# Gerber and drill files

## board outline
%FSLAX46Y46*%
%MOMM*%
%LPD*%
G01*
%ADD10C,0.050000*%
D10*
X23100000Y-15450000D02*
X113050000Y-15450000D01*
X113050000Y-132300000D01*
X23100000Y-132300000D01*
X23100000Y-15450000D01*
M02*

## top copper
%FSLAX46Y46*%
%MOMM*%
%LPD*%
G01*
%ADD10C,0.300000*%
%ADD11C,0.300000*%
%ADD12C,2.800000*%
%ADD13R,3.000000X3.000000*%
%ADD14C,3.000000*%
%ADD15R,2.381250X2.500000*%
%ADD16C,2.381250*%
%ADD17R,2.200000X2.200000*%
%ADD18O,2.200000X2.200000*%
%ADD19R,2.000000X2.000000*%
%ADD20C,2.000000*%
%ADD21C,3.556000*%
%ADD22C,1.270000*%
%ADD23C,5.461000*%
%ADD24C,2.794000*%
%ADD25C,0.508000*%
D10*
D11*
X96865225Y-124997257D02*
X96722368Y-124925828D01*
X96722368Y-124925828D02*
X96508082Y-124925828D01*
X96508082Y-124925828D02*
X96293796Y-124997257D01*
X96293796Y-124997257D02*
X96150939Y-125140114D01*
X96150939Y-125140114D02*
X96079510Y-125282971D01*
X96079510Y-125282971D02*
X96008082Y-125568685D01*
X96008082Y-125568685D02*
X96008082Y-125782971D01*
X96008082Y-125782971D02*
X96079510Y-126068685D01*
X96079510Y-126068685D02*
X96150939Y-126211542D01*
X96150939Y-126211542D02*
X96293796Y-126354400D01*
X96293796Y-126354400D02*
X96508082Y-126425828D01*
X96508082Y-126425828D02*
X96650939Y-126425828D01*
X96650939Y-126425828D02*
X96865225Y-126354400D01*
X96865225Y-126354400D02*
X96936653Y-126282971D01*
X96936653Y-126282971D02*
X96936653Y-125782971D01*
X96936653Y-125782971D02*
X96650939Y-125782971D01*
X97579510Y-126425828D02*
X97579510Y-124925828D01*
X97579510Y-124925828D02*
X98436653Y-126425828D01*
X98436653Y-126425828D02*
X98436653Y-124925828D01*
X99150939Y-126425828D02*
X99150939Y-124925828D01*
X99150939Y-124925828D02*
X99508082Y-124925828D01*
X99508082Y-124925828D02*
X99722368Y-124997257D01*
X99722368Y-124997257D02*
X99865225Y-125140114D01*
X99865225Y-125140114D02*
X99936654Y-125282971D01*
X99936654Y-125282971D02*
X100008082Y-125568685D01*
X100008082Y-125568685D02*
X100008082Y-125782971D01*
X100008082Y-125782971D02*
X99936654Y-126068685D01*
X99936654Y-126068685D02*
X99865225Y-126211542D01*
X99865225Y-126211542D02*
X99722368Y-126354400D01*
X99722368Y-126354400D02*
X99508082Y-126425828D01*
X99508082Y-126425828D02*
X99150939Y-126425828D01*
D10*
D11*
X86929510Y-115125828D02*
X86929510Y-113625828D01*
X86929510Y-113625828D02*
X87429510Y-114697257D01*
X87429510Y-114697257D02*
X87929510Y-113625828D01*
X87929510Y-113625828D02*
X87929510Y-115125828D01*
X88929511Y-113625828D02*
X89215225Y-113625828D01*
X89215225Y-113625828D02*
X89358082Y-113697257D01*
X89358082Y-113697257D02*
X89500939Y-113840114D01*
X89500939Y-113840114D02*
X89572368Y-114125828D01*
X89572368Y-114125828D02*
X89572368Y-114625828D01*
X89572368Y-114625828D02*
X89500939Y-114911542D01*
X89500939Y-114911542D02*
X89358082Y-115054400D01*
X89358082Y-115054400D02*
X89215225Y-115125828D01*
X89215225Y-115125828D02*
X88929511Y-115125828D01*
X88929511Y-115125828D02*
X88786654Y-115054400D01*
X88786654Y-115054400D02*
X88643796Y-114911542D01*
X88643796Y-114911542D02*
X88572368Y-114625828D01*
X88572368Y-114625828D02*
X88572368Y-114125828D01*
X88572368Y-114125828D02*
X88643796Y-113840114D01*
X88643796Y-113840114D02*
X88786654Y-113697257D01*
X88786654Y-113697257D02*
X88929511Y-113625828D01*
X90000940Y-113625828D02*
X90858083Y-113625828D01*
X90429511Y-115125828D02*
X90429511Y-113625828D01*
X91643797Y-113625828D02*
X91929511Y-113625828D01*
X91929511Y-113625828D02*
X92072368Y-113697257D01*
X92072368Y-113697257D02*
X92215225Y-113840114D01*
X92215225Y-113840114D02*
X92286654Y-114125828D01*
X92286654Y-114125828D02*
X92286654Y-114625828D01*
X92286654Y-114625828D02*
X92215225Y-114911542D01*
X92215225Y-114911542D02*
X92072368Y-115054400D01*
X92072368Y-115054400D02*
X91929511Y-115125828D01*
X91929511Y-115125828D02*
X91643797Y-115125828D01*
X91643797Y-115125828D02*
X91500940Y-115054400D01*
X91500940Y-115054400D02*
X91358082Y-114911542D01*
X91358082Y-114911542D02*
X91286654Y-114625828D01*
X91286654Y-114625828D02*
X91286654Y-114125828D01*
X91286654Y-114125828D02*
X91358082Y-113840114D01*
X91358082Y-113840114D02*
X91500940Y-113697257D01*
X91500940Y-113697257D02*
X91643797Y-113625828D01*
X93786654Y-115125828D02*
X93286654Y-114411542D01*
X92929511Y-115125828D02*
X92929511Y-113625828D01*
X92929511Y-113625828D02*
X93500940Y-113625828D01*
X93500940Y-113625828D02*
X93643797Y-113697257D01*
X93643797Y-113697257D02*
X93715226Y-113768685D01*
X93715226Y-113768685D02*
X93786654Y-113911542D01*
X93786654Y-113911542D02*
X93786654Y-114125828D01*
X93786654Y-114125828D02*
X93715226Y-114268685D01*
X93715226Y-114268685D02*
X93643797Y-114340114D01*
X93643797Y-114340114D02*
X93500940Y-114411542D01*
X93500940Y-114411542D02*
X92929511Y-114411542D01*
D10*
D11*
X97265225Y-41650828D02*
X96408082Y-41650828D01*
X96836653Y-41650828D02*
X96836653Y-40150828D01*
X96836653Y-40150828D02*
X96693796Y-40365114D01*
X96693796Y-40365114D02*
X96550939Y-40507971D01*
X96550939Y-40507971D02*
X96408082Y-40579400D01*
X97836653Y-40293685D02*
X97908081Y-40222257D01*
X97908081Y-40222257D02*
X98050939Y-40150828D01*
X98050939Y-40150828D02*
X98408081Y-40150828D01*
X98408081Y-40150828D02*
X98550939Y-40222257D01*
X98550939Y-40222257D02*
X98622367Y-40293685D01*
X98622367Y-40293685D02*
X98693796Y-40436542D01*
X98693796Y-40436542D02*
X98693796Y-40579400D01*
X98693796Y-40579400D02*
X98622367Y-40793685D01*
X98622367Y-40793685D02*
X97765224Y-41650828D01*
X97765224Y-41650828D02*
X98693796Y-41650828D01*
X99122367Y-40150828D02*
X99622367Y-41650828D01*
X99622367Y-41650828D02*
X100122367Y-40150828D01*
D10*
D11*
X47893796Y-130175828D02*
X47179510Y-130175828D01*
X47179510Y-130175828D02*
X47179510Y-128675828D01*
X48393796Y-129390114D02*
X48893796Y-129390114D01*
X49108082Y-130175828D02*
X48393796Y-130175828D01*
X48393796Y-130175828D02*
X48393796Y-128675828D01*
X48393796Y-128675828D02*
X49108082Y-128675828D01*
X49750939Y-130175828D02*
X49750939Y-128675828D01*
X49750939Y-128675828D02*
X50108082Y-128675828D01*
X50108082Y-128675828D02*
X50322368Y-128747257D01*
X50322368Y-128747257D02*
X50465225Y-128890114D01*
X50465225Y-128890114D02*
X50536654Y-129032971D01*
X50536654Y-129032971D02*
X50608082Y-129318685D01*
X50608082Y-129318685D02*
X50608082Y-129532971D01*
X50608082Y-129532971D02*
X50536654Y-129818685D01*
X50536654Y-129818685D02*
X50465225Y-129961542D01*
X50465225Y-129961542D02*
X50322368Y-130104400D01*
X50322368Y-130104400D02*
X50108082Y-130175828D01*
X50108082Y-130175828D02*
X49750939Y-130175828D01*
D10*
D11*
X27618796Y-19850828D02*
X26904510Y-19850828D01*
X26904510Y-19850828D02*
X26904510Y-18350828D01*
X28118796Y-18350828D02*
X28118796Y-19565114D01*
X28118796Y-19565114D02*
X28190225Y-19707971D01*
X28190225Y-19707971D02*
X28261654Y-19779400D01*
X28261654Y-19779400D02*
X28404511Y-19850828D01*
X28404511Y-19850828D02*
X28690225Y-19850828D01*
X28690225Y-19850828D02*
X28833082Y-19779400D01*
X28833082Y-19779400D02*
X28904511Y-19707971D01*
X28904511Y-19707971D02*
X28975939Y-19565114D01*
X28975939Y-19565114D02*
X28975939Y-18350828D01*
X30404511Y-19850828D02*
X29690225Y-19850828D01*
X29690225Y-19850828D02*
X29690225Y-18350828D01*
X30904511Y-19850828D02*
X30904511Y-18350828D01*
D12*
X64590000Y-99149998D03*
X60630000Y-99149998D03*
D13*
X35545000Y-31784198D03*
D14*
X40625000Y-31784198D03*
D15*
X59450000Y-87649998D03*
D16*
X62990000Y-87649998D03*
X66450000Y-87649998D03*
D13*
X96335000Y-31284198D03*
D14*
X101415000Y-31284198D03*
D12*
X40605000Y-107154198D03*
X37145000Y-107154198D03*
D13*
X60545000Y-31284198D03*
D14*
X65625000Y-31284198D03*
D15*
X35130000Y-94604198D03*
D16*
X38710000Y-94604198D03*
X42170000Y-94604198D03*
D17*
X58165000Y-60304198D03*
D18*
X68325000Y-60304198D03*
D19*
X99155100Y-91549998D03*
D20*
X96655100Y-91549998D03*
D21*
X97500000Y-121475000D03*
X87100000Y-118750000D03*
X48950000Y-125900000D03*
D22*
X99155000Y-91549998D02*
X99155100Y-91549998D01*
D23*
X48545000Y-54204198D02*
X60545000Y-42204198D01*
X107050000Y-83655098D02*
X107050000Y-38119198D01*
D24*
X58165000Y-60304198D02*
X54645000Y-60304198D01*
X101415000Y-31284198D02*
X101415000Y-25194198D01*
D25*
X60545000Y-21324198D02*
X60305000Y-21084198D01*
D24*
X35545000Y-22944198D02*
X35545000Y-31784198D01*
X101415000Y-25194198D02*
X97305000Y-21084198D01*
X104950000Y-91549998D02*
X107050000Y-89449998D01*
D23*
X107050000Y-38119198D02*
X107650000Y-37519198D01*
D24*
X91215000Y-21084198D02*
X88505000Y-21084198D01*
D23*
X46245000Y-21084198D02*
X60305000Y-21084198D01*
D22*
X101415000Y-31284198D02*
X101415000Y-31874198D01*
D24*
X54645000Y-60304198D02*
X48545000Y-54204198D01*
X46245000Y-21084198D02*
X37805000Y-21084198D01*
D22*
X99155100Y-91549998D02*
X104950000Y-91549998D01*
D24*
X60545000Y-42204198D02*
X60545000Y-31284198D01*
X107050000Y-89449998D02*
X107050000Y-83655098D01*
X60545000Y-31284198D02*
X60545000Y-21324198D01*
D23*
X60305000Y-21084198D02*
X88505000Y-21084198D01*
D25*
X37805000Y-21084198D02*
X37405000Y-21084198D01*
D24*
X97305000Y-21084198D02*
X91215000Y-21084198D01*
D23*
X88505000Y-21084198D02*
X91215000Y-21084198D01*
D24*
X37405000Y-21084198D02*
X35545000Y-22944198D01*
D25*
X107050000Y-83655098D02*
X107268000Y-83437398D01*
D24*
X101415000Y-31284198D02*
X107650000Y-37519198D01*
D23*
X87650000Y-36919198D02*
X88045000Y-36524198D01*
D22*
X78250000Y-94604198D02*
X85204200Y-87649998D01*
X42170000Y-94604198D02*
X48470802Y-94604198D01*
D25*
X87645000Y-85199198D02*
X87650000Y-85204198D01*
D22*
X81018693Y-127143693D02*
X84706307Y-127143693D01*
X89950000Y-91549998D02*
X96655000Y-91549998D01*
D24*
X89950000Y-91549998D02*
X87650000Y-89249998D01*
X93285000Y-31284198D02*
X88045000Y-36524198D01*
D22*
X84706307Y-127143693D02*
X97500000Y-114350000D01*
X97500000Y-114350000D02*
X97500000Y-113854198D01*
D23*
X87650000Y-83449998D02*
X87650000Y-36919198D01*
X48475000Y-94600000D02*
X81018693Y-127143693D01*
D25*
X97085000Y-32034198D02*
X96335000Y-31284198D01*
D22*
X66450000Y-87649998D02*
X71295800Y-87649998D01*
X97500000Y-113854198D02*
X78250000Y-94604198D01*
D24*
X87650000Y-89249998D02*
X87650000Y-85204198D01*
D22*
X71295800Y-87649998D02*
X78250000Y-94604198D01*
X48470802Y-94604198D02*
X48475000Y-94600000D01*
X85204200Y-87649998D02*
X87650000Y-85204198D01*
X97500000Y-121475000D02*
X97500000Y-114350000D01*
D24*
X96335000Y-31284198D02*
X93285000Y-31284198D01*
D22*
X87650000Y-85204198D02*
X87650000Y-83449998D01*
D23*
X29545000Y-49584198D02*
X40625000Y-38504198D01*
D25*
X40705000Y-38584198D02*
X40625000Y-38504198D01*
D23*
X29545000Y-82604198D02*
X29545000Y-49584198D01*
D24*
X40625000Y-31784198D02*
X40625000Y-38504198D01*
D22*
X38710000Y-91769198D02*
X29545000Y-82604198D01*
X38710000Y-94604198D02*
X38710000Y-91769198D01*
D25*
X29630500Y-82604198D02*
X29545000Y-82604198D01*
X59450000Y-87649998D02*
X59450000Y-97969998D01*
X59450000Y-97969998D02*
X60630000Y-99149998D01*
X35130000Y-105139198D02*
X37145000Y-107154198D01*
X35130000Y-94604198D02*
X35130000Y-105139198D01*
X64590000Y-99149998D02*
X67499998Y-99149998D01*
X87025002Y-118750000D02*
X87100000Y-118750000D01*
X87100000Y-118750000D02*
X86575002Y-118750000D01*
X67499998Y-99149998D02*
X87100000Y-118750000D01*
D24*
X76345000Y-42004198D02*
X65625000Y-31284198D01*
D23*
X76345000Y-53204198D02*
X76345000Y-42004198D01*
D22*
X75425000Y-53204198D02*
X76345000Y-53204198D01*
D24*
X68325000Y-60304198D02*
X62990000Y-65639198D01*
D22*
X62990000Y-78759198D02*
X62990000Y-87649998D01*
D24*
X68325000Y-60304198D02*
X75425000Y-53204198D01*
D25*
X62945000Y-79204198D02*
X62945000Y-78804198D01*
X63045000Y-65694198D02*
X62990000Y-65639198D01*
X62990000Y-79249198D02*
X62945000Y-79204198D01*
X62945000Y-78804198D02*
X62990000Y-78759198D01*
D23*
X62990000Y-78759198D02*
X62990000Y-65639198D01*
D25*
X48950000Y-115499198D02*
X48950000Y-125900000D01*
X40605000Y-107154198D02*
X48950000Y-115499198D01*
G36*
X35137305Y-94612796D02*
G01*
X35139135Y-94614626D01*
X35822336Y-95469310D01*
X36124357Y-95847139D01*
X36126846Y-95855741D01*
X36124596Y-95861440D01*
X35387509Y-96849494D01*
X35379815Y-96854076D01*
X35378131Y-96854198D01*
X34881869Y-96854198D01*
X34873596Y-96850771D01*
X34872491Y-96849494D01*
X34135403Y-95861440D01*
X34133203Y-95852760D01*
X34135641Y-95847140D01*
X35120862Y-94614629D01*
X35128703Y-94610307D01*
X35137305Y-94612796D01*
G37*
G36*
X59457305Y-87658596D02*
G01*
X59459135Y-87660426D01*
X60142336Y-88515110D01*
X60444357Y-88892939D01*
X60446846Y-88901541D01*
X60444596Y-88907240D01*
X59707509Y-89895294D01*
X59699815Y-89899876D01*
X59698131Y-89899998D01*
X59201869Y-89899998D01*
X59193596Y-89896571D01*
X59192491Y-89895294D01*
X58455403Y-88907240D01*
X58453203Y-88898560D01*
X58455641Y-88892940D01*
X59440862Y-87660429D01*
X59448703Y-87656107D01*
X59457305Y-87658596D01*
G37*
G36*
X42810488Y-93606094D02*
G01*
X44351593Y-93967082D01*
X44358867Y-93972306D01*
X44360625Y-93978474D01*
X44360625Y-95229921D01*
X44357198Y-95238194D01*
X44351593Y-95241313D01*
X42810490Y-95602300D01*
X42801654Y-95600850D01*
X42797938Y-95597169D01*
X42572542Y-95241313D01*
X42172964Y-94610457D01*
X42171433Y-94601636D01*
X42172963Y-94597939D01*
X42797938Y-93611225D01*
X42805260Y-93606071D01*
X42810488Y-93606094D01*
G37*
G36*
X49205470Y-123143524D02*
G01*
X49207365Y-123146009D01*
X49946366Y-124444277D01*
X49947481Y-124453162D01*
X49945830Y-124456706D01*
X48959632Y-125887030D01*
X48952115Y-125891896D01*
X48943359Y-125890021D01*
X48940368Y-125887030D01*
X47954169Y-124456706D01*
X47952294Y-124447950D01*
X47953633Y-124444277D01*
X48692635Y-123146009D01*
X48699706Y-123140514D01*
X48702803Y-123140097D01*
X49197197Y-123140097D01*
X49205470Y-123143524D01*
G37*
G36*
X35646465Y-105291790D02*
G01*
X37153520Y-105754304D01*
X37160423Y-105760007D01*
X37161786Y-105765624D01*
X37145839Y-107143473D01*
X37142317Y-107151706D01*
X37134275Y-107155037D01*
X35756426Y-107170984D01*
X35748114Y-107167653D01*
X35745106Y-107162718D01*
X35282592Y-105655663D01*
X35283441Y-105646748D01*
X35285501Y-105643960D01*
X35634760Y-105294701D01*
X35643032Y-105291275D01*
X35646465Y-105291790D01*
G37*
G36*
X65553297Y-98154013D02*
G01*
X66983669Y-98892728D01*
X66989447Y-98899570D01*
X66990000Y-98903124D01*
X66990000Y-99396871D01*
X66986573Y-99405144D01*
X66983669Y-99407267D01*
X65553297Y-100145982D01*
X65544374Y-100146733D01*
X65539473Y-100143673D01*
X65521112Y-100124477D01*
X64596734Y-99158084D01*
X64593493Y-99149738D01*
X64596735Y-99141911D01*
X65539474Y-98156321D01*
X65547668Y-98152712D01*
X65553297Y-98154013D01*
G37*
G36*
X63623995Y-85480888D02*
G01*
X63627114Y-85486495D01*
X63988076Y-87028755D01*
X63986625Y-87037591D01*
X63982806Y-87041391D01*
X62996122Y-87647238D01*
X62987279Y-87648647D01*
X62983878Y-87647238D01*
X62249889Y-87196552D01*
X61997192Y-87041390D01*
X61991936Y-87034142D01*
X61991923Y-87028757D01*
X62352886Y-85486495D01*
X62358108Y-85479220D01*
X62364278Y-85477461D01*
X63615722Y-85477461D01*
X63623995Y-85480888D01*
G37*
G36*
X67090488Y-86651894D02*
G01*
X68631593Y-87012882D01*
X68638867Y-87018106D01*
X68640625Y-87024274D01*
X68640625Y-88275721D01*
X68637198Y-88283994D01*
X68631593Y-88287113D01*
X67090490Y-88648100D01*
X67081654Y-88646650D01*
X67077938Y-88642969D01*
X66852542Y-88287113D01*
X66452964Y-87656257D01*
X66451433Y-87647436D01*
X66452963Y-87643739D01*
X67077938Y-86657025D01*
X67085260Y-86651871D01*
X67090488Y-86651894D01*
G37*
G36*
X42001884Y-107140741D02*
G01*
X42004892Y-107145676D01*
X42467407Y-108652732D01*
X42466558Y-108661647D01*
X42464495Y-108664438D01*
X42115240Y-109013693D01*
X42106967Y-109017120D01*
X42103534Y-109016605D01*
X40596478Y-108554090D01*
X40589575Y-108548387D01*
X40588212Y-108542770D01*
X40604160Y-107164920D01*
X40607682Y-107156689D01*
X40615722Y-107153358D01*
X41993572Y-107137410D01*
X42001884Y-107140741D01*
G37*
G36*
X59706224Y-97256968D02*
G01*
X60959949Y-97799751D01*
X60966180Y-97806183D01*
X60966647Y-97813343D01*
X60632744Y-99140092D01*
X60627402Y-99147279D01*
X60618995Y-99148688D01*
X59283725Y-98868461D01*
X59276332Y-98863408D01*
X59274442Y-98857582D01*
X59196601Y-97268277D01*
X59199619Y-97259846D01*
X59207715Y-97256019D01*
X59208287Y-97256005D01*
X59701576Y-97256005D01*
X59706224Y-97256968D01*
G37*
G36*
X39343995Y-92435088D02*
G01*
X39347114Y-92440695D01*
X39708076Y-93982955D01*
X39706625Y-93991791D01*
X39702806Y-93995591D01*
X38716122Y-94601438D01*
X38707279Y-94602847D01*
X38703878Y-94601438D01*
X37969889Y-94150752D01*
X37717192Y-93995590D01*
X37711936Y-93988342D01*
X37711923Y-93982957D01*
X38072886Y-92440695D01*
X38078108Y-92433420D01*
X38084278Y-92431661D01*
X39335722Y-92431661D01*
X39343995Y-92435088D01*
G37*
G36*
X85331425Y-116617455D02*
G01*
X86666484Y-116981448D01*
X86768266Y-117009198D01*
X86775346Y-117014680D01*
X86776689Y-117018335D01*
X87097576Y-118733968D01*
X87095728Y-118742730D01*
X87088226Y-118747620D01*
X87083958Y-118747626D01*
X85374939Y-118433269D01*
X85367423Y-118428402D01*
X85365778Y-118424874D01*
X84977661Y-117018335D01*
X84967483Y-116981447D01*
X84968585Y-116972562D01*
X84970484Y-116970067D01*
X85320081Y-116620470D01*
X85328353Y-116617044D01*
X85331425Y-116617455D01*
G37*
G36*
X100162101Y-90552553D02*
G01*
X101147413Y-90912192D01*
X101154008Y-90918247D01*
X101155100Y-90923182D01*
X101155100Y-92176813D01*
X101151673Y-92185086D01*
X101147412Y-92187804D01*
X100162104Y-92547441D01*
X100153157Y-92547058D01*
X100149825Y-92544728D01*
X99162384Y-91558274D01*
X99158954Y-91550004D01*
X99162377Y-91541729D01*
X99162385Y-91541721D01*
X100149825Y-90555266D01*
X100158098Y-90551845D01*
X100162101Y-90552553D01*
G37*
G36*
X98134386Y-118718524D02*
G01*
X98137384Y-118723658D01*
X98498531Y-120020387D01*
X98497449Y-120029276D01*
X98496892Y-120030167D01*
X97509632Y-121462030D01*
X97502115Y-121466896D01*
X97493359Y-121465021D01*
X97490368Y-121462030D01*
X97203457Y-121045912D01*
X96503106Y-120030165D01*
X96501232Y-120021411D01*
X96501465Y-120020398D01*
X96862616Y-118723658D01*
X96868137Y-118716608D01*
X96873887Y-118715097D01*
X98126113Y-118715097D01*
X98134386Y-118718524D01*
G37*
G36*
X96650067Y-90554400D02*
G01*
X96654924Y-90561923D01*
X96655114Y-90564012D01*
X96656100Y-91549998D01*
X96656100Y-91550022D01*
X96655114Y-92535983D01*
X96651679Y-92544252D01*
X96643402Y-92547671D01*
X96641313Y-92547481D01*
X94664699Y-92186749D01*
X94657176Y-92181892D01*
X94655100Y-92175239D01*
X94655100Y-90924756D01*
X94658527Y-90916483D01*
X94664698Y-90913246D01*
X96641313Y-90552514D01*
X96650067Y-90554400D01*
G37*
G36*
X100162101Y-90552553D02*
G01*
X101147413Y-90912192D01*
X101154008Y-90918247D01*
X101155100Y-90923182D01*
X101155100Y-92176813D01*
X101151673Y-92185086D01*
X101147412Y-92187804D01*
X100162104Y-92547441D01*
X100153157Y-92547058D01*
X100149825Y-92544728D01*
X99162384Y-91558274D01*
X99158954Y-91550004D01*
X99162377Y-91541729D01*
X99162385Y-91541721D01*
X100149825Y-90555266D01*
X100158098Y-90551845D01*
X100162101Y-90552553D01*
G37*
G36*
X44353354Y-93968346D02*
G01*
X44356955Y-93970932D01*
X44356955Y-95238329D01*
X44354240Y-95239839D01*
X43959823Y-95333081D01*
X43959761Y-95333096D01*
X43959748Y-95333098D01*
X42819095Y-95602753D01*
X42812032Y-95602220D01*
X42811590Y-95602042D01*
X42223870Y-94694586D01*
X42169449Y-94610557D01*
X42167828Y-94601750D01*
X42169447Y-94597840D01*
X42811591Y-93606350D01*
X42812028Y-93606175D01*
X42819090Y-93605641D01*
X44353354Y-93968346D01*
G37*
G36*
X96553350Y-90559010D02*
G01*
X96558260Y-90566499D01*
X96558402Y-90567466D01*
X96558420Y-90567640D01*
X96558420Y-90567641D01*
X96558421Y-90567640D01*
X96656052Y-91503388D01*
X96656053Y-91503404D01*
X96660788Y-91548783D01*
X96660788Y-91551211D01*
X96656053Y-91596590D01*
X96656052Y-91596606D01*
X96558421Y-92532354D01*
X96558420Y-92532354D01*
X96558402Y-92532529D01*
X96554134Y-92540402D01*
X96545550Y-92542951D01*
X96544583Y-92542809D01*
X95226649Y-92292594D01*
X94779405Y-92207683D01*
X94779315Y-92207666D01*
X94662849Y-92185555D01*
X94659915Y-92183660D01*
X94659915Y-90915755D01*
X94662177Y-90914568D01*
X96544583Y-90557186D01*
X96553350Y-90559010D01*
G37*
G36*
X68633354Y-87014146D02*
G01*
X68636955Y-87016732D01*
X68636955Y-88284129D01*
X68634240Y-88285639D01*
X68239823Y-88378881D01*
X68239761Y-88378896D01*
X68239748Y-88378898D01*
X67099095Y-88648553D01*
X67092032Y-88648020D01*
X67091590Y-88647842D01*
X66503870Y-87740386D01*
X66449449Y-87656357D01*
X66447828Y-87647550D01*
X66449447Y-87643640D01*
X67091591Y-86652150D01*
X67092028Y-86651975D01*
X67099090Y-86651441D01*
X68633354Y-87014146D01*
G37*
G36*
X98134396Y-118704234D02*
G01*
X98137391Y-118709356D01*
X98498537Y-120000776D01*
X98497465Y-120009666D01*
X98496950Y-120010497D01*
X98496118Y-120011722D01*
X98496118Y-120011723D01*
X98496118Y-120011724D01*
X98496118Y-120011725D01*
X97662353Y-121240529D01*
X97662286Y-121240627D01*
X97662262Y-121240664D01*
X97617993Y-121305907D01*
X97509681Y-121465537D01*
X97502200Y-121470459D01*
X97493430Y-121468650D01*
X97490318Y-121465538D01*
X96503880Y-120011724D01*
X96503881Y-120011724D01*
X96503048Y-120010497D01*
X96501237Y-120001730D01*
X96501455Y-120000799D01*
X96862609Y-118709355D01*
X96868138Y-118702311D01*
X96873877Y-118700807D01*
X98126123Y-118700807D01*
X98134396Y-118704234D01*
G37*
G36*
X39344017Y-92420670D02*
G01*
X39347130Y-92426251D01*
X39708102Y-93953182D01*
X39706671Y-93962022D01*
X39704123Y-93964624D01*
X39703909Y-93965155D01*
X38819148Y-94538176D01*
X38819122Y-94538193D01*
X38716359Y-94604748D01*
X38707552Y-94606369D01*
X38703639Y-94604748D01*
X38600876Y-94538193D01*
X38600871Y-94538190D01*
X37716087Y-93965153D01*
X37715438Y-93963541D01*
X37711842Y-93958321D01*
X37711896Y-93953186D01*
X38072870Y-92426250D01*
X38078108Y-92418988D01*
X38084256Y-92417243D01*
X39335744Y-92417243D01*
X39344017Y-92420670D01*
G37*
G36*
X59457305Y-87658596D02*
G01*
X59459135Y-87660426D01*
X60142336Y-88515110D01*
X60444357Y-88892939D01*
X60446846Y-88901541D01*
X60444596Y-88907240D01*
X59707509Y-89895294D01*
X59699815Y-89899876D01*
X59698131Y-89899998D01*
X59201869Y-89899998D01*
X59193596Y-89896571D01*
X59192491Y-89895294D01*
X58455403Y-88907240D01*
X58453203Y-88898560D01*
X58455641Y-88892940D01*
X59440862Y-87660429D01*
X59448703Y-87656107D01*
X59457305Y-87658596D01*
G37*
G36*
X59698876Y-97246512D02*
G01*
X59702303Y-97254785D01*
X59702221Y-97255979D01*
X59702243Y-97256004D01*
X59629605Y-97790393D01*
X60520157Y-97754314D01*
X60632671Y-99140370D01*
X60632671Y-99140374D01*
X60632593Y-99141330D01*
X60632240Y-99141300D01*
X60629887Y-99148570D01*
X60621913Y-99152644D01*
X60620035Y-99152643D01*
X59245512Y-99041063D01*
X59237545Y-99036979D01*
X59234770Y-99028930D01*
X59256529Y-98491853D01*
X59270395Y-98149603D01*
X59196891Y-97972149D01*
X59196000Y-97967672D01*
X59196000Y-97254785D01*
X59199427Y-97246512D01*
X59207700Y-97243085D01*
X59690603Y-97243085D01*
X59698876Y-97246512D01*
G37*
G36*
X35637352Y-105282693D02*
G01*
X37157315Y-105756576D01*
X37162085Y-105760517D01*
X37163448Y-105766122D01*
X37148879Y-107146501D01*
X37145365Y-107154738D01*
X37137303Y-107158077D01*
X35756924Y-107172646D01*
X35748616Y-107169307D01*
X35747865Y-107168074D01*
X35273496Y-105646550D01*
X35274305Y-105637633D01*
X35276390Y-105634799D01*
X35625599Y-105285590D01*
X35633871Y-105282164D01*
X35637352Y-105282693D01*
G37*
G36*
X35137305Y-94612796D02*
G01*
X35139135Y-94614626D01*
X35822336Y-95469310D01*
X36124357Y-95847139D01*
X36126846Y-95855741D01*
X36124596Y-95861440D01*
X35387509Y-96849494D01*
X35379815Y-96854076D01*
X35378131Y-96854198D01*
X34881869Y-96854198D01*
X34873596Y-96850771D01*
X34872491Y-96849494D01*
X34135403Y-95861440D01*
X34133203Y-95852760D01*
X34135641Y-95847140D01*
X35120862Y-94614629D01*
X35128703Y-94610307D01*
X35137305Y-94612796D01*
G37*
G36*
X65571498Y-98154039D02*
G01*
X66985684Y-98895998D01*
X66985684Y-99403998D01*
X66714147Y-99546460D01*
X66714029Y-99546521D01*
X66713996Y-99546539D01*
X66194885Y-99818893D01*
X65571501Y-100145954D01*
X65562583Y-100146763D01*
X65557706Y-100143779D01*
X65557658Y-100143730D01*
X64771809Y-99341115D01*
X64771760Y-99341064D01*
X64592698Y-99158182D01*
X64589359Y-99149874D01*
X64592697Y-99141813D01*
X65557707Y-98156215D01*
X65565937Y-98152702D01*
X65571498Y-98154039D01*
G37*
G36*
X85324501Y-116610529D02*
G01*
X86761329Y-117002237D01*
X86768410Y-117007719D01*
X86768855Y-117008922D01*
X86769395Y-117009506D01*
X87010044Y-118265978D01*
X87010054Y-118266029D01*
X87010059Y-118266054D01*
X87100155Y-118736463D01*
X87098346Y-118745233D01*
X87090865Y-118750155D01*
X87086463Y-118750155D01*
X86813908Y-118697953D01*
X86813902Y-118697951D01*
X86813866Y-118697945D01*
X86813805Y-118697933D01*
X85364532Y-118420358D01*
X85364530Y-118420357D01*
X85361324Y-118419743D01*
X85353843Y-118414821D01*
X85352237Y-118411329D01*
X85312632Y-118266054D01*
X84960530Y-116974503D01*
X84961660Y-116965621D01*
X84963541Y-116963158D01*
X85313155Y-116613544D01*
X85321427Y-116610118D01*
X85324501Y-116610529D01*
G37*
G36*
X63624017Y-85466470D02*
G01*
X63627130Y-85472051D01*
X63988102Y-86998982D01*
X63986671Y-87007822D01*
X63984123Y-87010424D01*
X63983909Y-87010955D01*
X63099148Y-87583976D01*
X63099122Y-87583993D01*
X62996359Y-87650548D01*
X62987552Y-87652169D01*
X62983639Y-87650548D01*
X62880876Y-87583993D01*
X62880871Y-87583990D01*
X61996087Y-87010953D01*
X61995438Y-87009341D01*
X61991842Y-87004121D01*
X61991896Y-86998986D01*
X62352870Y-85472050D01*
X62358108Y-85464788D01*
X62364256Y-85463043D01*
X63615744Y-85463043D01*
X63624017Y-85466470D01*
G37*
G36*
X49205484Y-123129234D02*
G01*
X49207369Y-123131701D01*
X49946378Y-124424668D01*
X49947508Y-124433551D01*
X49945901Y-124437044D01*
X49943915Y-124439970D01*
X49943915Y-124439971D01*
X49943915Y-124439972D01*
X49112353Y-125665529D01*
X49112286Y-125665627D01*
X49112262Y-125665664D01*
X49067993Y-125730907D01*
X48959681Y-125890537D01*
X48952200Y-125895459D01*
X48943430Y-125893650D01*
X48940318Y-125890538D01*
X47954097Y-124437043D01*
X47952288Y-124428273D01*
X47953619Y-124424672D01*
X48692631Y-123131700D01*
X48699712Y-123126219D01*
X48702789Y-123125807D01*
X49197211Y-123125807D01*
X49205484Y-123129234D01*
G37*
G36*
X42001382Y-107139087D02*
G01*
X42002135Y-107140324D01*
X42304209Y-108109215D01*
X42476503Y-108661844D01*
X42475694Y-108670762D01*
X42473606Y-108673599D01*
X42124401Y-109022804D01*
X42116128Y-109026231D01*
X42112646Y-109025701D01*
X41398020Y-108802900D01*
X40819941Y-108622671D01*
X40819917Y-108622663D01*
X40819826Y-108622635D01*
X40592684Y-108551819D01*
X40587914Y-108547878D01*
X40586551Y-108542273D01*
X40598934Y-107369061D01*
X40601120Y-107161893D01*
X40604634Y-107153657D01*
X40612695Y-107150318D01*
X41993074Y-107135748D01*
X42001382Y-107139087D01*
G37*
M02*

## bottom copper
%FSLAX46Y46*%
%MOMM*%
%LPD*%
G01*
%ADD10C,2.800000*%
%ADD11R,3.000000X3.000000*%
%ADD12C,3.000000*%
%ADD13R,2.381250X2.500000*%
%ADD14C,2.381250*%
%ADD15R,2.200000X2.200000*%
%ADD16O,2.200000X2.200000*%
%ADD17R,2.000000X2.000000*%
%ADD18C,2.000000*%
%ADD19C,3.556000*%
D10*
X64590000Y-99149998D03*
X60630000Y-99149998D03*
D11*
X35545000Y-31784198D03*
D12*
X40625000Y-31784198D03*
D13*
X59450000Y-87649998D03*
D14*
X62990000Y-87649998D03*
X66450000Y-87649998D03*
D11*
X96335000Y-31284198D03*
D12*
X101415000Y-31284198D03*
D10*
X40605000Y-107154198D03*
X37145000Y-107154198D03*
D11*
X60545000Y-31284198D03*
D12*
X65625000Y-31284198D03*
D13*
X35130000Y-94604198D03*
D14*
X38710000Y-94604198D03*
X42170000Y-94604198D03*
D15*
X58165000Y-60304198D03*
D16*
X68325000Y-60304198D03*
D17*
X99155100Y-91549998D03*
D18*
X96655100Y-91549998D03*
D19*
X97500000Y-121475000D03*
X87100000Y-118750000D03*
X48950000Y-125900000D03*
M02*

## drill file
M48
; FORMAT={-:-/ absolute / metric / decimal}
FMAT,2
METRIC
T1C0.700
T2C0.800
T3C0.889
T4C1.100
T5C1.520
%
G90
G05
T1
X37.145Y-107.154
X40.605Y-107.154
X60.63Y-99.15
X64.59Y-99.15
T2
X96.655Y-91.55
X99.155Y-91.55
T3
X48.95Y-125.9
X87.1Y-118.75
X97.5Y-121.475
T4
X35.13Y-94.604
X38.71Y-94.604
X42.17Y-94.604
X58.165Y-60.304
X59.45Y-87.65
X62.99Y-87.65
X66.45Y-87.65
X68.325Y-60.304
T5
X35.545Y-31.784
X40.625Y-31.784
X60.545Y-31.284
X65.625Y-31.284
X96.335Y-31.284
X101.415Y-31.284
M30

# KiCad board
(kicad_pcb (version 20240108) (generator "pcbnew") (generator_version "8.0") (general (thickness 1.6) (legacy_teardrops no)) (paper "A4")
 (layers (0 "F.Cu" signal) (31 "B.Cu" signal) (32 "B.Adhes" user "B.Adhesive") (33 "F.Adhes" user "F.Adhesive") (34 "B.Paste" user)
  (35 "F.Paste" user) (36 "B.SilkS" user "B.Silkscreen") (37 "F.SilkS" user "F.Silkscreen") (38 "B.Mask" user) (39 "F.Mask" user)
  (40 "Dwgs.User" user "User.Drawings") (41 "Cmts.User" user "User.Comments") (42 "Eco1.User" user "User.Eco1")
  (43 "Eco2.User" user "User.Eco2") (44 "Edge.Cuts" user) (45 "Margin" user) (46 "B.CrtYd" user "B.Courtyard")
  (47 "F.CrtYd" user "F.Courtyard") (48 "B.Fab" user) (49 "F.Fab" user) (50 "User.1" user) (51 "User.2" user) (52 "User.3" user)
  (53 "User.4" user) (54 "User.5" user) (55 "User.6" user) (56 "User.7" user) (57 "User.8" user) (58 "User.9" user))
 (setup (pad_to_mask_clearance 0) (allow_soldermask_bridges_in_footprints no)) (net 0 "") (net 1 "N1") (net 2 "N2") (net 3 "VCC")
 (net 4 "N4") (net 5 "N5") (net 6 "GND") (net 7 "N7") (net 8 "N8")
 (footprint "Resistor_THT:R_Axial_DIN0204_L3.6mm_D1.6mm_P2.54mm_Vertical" (layer "F.Cu") (at 63.17 99.149998 180)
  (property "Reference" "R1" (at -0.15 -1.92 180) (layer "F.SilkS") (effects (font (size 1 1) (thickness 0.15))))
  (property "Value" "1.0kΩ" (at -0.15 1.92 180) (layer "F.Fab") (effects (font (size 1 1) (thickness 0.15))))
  (pad "1" thru_hole circle (at -1.42 0 180) (size 2.8 2.8) (drill 0.7) (layers "*.Cu" "*.Mask") (remove_unused_layers no) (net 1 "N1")
   (teardrops (best_length_ratio 0.5) (max_length 1) (best_width_ratio 1) (max_width 2) (curve_points 0) (filter_ratio 0.9) (enabled yes)
    (allow_two_segments yes) (prefer_zone_connections yes)))
  (pad "2" thru_hole circle (at 2.54 0 180) (size 2.8 2.8) (drill 0.7) (layers "*.Cu" "*.Mask") (remove_unused_layers no) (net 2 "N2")
   (teardrops (best_length_ratio 0.5) (max_length 1) (best_width_ratio 1) (max_width 2) (curve_points 0) (filter_ratio 0.9) (enabled yes)
    (allow_two_segments yes) (prefer_zone_connections yes))))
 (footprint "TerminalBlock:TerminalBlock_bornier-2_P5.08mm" (layer "F.Cu") (at 35.545 31.784198)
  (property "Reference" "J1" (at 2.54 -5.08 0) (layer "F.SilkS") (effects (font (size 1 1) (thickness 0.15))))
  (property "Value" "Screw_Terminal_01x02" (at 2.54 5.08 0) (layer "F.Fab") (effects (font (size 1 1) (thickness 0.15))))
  (pad "1" thru_hole rect (at 0 0) (size 3 3) (drill 1.52) (layers "*.Cu" "*.Mask") (remove_unused_layers no) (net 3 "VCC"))
  (pad "2" thru_hole circle (at 5.08 0) (size 3 3) (drill 1.52) (layers "*.Cu" "*.Mask") (remove_unused_layers no) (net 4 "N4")))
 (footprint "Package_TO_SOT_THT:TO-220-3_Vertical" (layer "F.Cu") (at 60.45 87.649998)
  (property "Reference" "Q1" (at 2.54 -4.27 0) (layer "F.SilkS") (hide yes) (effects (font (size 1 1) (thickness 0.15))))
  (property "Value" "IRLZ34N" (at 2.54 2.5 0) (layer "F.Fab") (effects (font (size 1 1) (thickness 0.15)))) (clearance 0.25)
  (pad "1" thru_hole rect (at -1 0) (size 2.38125 2.5) (drill 1.1) (layers "*.Cu" "*.Mask") (remove_unused_layers no) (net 2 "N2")
   (teardrops (best_length_ratio 0.5) (max_length 1) (best_width_ratio 1) (max_width 2) (curve_points 0) (filter_ratio 0.9) (enabled yes)
    (allow_two_segments yes) (prefer_zone_connections yes)))
  (pad "2" thru_hole circle (at 2.54 0) (size 2.38125 2.38125) (drill 1.1) (layers "*.Cu" "*.Mask") (remove_unused_layers no) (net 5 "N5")
   (clearance 0.2)
   (teardrops (best_length_ratio 0.5) (max_length 1) (best_width_ratio 1) (max_width 2) (curve_points 0) (filter_ratio 0.9) (enabled yes)
    (allow_two_segments yes) (prefer_zone_connections yes)))
  (pad "3" thru_hole circle (at 6 0) (size 2.38125 2.38125) (drill 1.1) (layers "*.Cu" "*.Mask") (remove_unused_layers no) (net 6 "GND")
   (teardrops (best_length_ratio 0.5) (max_length 1) (best_width_ratio 1) (max_width 2) (curve_points 0) (filter_ratio 0.9) (enabled yes)
    (allow_two_segments yes) (prefer_zone_connections yes))))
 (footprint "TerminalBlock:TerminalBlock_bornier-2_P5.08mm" (layer "F.Cu") (at 96.335 31.284198)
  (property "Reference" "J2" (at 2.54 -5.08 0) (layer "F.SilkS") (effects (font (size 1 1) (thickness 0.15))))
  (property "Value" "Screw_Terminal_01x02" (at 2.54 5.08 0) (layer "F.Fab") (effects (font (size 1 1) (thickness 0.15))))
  (pad "1" thru_hole rect (at 0 0) (size 3 3) (drill 1.52) (layers "*.Cu" "*.Mask") (remove_unused_layers no) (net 6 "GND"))
  (pad "2" thru_hole circle (at 5.08 0) (size 3 3) (drill 1.52) (layers "*.Cu" "*.Mask") (remove_unused_layers no) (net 3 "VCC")))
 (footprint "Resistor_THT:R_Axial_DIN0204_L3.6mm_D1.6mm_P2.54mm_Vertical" (layer "F.Cu") (at 39.685 107.154198 180)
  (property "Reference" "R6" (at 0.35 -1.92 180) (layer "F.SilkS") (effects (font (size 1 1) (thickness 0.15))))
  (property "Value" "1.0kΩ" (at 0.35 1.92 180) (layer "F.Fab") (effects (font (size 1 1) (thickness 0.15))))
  (pad "1" thru_hole circle (at -0.92 0 180) (size 2.8 2.8) (drill 0.7) (layers "*.Cu" "*.Mask") (remove_unused_layers no) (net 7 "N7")
   (teardrops (best_length_ratio 0.5) (max_length 1) (best_width_ratio 1) (max_width 2) (curve_points 0) (filter_ratio 0.9) (enabled yes)
    (allow_two_segments yes) (prefer_zone_connections yes)))
  (pad "2" thru_hole circle (at 2.54 0 180) (size 2.8 2.8) (drill 0.7) (layers "*.Cu" "*.Mask") (remove_unused_layers no) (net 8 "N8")
   (teardrops (best_length_ratio 0.5) (max_length 1) (best_width_ratio 1) (max_width 2) (curve_points 0) (filter_ratio 0.9) (enabled yes)
    (allow_two_segments yes) (prefer_zone_connections yes))))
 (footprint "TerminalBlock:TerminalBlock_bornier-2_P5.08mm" (layer "F.Cu") (at 60.545 31.284198)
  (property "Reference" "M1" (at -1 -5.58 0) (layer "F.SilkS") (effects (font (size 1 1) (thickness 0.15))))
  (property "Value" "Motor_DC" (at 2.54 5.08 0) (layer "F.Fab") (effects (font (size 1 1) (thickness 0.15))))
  (pad "1" thru_hole rect (at 0 0) (size 3 3) (drill 1.52) (layers "*.Cu" "*.Mask") (remove_unused_layers no) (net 3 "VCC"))
  (pad "2" thru_hole circle (at 5.08 0) (size 3 3) (drill 1.52) (layers "*.Cu" "*.Mask") (remove_unused_layers no) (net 5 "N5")))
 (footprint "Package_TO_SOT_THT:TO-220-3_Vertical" (layer "F.Cu") (at 37.17 94.604198)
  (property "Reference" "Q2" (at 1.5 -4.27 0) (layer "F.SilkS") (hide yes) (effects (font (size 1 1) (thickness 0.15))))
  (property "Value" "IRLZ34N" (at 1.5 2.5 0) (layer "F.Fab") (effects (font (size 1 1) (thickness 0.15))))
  (pad "1" thru_hole rect (at -2.04 0) (size 2.38125 2.5) (drill 1.1) (layers "*.Cu" "*.Mask") (remove_unused_layers no) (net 8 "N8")
   (teardrops (best_length_ratio 0.5) (max_length 1) (best_width_ratio 1) (max_width 2) (curve_points 0) (filter_ratio 0.9) (enabled yes)
    (allow_two_segments yes) (prefer_zone_connections yes)))
  (pad "2" thru_hole circle (at 1.54 0) (size 2.38125 2.38125) (drill 1.1) (layers "*.Cu" "*.Mask") (remove_unused_layers no) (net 4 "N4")
   (teardrops (best_length_ratio 0.5) (max_length 1) (best_width_ratio 1) (max_width 2) (curve_points 0) (filter_ratio 0.9) (enabled yes)
    (allow_two_segments yes) (prefer_zone_connections yes)))
  (pad "3" thru_hole circle (at 5 0) (size 2.38125 2.38125) (drill 1.1) (layers "*.Cu" "*.Mask") (remove_unused_layers no) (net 6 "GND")
   (teardrops (best_length_ratio 0.5) (max_length 1) (best_width_ratio 1) (max_width 2) (curve_points 0) (filter_ratio 0.9) (enabled yes)
    (allow_two_segments yes) (prefer_zone_connections yes))))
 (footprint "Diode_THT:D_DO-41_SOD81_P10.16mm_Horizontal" (layer "F.Cu") (at 58.165 60.304198)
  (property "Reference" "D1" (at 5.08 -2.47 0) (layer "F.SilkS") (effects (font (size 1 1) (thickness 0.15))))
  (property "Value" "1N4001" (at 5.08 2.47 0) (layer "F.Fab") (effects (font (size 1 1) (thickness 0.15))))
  (pad "1" thru_hole rect (at 0 0) (size 2.2 2.2) (drill 1.1) (layers "*.Cu" "*.Mask") (remove_unused_layers no) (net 3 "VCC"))
  (pad "2" thru_hole oval (at 10.16 0) (size 2.2 2.2) (drill 1.1) (layers "*.Cu" "*.Mask") (remove_unused_layers no) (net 5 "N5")))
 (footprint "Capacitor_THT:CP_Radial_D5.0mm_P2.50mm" (layer "F.Cu") (at 99.1551 91.549998 180)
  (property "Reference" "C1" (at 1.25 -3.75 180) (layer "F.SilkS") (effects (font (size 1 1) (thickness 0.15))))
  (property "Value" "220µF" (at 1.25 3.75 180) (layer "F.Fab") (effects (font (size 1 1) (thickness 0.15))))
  (pad "1" thru_hole rect (at 0 0 180) (size 2 2) (drill 0.8) (layers "*.Cu" "*.Mask") (remove_unused_layers no) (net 3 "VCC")
   (teardrops (best_length_ratio 0.5) (max_length 1) (best_width_ratio 1) (max_width 2) (curve_points 0) (filter_ratio 0.9) (enabled yes)
    (allow_two_segments yes) (prefer_zone_connections yes)))
  (pad "2" thru_hole circle (at 2.5 0 180) (size 2 2) (drill 0.8) (layers "*.Cu" "*.Mask") (remove_unused_layers no) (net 6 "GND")
   (teardrops (best_length_ratio 0.5) (max_length 1) (best_width_ratio 1) (max_width 2) (curve_points 0) (filter_ratio 0.9) (enabled yes)
    (allow_two_segments yes) (prefer_zone_connections yes))))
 (gr_rect (start 23.1 15.45) (end 113.05 132.3) (stroke (width 0.05) (type default)) (fill none) (layer "Edge.Cuts"))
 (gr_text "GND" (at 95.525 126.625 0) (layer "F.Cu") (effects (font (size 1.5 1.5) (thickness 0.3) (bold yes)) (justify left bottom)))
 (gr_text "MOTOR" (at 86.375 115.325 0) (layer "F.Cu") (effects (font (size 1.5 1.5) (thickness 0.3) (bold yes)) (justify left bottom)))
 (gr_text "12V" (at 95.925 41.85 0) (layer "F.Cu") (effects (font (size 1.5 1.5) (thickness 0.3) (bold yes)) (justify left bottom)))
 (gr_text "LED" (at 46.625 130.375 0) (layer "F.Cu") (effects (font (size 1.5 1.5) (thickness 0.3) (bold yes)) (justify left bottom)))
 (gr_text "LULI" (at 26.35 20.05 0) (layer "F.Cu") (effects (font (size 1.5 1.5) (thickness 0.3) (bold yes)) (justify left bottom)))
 (segment (start 99.155 91.549998) (end 99.1551 91.549998) (width 1.27) (layer "F.Cu") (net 3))
 (segment (start 48.545 54.204198) (end 60.545 42.204198) (width 5.461) (layer "F.Cu") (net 3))
 (segment (start 107.05 83.655098) (end 107.05 38.119198) (width 5.461) (layer "F.Cu") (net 3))
 (segment (start 58.165 60.304198) (end 54.645 60.304198) (width 2.794) (layer "F.Cu") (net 3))
 (segment (start 101.415 31.284198) (end 101.415 25.194198) (width 2.794) (layer "F.Cu") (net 3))
 (segment (start 60.545 21.324198) (end 60.305 21.084198) (width 0.508) (layer "F.Cu") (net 3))
 (segment (start 35.545 22.944198) (end 35.545 31.784198) (width 2.794) (layer "F.Cu") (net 3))
 (segment (start 101.415 25.194198) (end 97.305 21.084198) (width 2.794) (layer "F.Cu") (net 3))
 (segment (start 104.95 91.549998) (end 107.05 89.449998) (width 2.794) (layer "F.Cu") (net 3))
 (segment (start 107.05 38.119198) (end 107.65 37.519198) (width 5.461) (layer "F.Cu") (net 3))
 (segment (start 91.215 21.084198) (end 88.505 21.084198) (width 2.794) (layer "F.Cu") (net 3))
 (segment (start 46.245 21.084198) (end 60.305 21.084198) (width 5.461) (layer "F.Cu") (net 3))
 (segment (start 101.415 31.284198) (end 101.415 31.874198) (width 1.27) (layer "F.Cu") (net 3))
 (segment (start 54.645 60.304198) (end 48.545 54.204198) (width 2.794) (layer "F.Cu") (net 3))
 (segment (start 46.245 21.084198) (end 37.805 21.084198) (width 2.794) (layer "F.Cu") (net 3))
 (segment (start 99.1551 91.549998) (end 104.95 91.549998) (width 1.27) (layer "F.Cu") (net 3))
 (segment (start 60.545 42.204198) (end 60.545 31.284198) (width 2.794) (layer "F.Cu") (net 3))
 (segment (start 107.05 89.449998) (end 107.05 83.655098) (width 2.794) (layer "F.Cu") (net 3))
 (segment (start 60.545 31.284198) (end 60.545 21.324198) (width 2.794) (layer "F.Cu") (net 3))
 (segment (start 60.305 21.084198) (end 88.505 21.084198) (width 5.461) (layer "F.Cu") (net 3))
 (segment (start 37.805 21.084198) (end 37.405 21.084198) (width 0.508) (layer "F.Cu") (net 3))
 (segment (start 97.305 21.084198) (end 91.215 21.084198) (width 2.794) (layer "F.Cu") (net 3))
 (segment (start 88.505 21.084198) (end 91.215 21.084198) (width 5.461) (layer "F.Cu") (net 3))
 (segment (start 37.405 21.084198) (end 35.545 22.944198) (width 2.794) (layer "F.Cu") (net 3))
 (segment (start 107.05 83.655098) (end 107.268 83.437398) (width 0.508) (layer "F.Cu") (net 3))
 (segment (start 101.415 31.284198) (end 107.65 37.519198) (width 2.794) (layer "F.Cu") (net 3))
 (segment (start 87.65 36.919198) (end 88.045 36.524198) (width 5.461) (layer "F.Cu") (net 6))
 (segment (start 78.25 94.604198) (end 85.2042 87.649998) (width 1.27) (layer "F.Cu") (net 6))
 (segment (start 42.17 94.604198) (end 48.470802 94.604198) (width 1.27) (layer "F.Cu") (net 6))
 (segment (start 87.645 85.199198) (end 87.65 85.204198) (width 0.508) (layer "F.Cu") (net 6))
 (segment (start 81.018693 127.143693) (end 84.706307 127.143693) (width 1.27) (layer "F.Cu") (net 6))
 (segment (start 89.95 91.549998) (end 96.655 91.549998) (width 1.27) (layer "F.Cu") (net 6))
 (segment (start 89.95 91.549998) (end 87.65 89.249998) (width 2.794) (layer "F.Cu") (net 6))
 (segment (start 93.285 31.284198) (end 88.045 36.524198) (width 2.794) (layer "F.Cu") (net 6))
 (segment (start 84.706307 127.143693) (end 97.5 114.35) (width 1.27) (layer "F.Cu") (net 6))
 (segment (start 97.5 114.35) (end 97.5 113.854198) (width 1.27) (layer "F.Cu") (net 6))
 (segment (start 87.65 83.449998) (end 87.65 36.919198) (width 5.461) (layer "F.Cu") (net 6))
 (segment (start 48.475 94.6) (end 81.018693 127.143693) (width 5.461) (layer "F.Cu") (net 6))
 (segment (start 97.085 32.034198) (end 96.335 31.284198) (width 0.508) (layer "F.Cu") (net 6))
 (segment (start 66.45 87.649998) (end 71.2958 87.649998) (width 1.27) (layer "F.Cu") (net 6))
 (segment (start 97.5 113.854198) (end 78.25 94.604198) (width 1.27) (layer "F.Cu") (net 6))
 (segment (start 87.65 89.249998) (end 87.65 85.204198) (width 2.794) (layer "F.Cu") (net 6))
 (segment (start 71.2958 87.649998) (end 78.25 94.604198) (width 1.27) (layer "F.Cu") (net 6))
 (segment (start 48.470802 94.604198) (end 48.475 94.6) (width 1.27) (layer "F.Cu") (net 6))
 (segment (start 85.2042 87.649998) (end 87.65 85.204198) (width 1.27) (layer "F.Cu") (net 6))
 (segment (start 97.5 121.475) (end 97.5 114.35) (width 1.27) (layer "F.Cu") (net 6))
 (segment (start 96.335 31.284198) (end 93.285 31.284198) (width 2.794) (layer "F.Cu") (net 6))
 (segment (start 87.65 85.204198) (end 87.65 83.449998) (width 1.27) (layer "F.Cu") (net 6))
 (via (at 97.5 121.475) (size 3.556) (drill 0.889) (layers "F.Cu" "B.Cu") (free yes)
  (teardrops (best_length_ratio 0.5) (max_length 1) (best_width_ratio 1) (max_width 2) (curve_points 0) (filter_ratio 0.9) (enabled yes)
   (allow_two_segments yes) (prefer_zone_connections yes))
  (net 6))
 (segment (start 29.545 49.584198) (end 40.625 38.504198) (width 5.461) (layer "F.Cu") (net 4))
 (segment (start 40.705 38.584198) (end 40.625 38.504198) (width 0.508) (layer "F.Cu") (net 4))
 (segment (start 29.545 82.604198) (end 29.545 49.584198) (width 5.461) (layer "F.Cu") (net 4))
 (segment (start 40.625 31.784198) (end 40.625 38.504198) (width 2.794) (layer "F.Cu") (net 4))
 (segment (start 38.71 91.769198) (end 29.545 82.604198) (width 1.27) (layer "F.Cu") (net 4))
 (segment (start 38.71 94.604198) (end 38.71 91.769198) (width 1.27) (layer "F.Cu") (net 4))
 (segment (start 29.6305 82.604198) (end 29.545 82.604198) (width 0.508) (layer "F.Cu") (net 4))
 (segment (start 59.45 87.649998) (end 59.45 97.969998) (width 0.508) (layer "F.Cu") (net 2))
 (segment (start 59.45 97.969998) (end 60.63 99.149998) (width 0.508) (layer "F.Cu") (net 2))
 (segment (start 35.13 105.139198) (end 37.145 107.154198) (width 0.508) (layer "F.Cu") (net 8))
 (segment (start 35.13 94.604198) (end 35.13 105.139198) (width 0.508) (layer "F.Cu") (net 8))
 (segment (start 64.59 99.149998) (end 67.499998 99.149998) (width 0.508) (layer "F.Cu") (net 1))
 (segment (start 87.025002 118.75) (end 87.1 118.75) (width 0.508) (layer "F.Cu") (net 1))
 (segment (start 87.1 118.75) (end 86.575002 118.75) (width 0.508) (layer "F.Cu") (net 1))
 (segment (start 67.499998 99.149998) (end 87.1 118.75) (width 0.508) (layer "F.Cu") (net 1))
 (via (at 87.1 118.75) (size 3.556) (drill 0.889) (layers "F.Cu" "B.Cu")
  (teardrops (best_length_ratio 0.5) (max_length 1) (best_width_ratio 1) (max_width 2) (curve_points 0) (filter_ratio 0.9) (enabled yes)
   (allow_two_segments yes) (prefer_zone_connections yes))
  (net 1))
 (segment (start 76.345 42.004198) (end 65.625 31.284198) (width 2.794) (layer "F.Cu") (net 5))
 (segment (start 76.345 53.204198) (end 76.345 42.004198) (width 5.461) (layer "F.Cu") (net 5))
 (segment (start 75.425 53.204198) (end 76.345 53.204198) (width 1.27) (layer "F.Cu") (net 5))
 (segment (start 68.325 60.304198) (end 62.99 65.639198) (width 2.794) (layer "F.Cu") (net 5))
 (segment (start 62.99 78.759198) (end 62.99 87.649998) (width 1.27) (layer "F.Cu") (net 5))
 (segment (start 68.325 60.304198) (end 75.425 53.204198) (width 2.794) (layer "F.Cu") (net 5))
 (segment (start 62.945 79.204198) (end 62.945 78.804198) (width 0.508) (layer "F.Cu") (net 5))
 (segment (start 63.045 65.694198) (end 62.99 65.639198) (width 0.508) (layer "F.Cu") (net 5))
 (segment (start 62.99 79.249198) (end 62.945 79.204198) (width 0.508) (layer "F.Cu") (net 5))
 (segment (start 62.945 78.804198) (end 62.99 78.759198) (width 0.508) (layer "F.Cu") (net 5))
 (segment (start 62.99 78.759198) (end 62.99 65.639198) (width 5.461) (layer "F.Cu") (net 5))
 (segment (start 48.95 115.499198) (end 48.95 125.9) (width 0.508) (layer "F.Cu") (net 7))
 (segment (start 40.605 107.154198) (end 48.95 115.499198) (width 0.508) (layer "F.Cu") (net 7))
 (via (at 48.95 125.9) (size 3.556) (drill 0.889) (layers "F.Cu" "B.Cu")
  (teardrops (best_length_ratio 0.5) (max_length 1) (best_width_ratio 1) (max_width 2) (curve_points 0) (filter_ratio 0.9) (enabled yes)
   (allow_two_segments yes) (prefer_zone_connections yes))
  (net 7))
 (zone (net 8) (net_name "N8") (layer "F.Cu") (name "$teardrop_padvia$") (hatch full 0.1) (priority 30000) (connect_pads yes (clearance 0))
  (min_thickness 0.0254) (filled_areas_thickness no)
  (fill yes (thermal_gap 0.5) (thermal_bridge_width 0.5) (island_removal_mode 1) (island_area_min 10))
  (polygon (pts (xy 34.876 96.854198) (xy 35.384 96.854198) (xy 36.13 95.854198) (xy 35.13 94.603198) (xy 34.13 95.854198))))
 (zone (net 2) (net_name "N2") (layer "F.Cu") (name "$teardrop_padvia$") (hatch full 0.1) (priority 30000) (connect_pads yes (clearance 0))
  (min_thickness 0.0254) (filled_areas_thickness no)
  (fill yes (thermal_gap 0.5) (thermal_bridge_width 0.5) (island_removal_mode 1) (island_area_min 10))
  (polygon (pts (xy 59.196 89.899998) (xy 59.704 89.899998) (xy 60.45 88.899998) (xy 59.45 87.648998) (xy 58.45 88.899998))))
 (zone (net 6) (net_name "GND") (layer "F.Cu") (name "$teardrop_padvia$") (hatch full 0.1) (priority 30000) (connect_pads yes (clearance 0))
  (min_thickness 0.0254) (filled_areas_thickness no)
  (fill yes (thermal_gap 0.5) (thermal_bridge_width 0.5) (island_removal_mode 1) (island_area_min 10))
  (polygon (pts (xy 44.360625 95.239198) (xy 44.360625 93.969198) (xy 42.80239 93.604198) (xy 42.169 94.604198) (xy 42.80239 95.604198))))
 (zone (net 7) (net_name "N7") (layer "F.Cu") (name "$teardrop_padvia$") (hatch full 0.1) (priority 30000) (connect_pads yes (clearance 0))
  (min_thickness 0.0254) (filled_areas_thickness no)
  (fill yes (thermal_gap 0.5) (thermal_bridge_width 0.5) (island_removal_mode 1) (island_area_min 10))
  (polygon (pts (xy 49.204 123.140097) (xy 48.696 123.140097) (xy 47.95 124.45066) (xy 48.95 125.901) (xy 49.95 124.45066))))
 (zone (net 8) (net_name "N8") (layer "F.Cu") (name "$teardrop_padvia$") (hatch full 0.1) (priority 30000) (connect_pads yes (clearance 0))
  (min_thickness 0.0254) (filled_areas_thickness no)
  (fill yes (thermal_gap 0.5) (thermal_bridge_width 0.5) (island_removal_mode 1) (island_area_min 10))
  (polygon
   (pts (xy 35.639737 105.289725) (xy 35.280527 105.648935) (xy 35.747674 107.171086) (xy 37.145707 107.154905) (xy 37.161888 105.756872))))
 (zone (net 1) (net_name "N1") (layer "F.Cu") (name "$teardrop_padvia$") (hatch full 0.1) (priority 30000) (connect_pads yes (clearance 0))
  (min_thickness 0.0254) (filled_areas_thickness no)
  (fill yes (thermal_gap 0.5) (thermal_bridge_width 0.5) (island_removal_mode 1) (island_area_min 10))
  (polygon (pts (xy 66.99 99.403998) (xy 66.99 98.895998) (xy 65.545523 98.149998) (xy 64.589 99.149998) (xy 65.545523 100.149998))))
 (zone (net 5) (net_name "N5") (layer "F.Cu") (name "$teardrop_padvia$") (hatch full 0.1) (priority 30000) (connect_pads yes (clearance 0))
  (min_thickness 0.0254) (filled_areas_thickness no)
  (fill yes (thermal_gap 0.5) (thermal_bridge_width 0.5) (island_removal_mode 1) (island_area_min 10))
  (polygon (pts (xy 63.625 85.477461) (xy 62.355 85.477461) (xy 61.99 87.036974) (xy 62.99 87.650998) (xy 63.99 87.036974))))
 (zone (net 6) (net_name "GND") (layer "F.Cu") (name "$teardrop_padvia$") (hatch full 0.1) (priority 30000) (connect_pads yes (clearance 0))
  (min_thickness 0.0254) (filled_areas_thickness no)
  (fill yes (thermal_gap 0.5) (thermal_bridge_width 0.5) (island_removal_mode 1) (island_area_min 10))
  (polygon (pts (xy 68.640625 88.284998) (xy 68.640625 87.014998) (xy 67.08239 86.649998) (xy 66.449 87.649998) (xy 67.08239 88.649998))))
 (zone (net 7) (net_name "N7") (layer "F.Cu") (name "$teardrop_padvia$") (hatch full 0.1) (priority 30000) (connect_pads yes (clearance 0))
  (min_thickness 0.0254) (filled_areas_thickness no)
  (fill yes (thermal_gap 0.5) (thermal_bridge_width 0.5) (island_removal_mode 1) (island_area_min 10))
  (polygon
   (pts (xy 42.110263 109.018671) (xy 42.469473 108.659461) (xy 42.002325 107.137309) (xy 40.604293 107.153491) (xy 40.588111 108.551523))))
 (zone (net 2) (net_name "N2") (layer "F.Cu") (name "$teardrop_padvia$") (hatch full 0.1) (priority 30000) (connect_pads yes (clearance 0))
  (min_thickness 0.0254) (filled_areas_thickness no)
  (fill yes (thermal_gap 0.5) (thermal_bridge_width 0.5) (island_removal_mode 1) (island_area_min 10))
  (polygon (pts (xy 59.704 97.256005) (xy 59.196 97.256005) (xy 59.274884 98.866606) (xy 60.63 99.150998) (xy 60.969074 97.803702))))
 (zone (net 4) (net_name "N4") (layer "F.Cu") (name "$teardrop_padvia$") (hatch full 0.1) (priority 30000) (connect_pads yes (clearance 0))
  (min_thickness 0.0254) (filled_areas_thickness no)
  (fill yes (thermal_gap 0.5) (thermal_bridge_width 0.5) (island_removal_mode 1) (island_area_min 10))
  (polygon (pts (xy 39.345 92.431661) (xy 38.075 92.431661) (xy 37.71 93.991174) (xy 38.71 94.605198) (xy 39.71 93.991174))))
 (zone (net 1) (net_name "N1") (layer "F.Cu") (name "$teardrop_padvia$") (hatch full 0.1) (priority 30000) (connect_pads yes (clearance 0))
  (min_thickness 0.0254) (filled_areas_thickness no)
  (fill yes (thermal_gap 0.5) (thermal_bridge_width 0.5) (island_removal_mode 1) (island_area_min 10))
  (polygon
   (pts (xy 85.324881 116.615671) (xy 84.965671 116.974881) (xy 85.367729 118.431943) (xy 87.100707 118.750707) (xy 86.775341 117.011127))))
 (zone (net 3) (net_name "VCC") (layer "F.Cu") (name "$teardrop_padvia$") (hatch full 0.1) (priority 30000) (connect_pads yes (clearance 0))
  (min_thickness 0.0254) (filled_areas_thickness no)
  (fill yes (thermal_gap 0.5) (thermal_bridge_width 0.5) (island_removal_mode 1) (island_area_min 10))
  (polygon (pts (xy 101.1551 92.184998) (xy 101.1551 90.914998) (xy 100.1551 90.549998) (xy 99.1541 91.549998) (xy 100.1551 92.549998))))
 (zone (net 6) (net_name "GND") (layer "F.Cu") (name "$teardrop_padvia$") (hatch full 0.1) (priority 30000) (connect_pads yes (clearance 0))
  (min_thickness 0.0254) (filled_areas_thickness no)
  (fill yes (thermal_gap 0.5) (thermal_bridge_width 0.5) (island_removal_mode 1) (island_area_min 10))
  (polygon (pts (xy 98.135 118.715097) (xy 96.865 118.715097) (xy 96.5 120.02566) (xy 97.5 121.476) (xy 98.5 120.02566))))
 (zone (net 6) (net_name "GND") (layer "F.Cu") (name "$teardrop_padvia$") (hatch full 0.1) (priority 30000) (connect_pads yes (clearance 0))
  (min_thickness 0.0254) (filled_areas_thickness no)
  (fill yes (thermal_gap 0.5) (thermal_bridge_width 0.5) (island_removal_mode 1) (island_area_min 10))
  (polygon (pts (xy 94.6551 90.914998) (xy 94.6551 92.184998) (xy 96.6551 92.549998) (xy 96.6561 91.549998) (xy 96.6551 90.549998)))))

